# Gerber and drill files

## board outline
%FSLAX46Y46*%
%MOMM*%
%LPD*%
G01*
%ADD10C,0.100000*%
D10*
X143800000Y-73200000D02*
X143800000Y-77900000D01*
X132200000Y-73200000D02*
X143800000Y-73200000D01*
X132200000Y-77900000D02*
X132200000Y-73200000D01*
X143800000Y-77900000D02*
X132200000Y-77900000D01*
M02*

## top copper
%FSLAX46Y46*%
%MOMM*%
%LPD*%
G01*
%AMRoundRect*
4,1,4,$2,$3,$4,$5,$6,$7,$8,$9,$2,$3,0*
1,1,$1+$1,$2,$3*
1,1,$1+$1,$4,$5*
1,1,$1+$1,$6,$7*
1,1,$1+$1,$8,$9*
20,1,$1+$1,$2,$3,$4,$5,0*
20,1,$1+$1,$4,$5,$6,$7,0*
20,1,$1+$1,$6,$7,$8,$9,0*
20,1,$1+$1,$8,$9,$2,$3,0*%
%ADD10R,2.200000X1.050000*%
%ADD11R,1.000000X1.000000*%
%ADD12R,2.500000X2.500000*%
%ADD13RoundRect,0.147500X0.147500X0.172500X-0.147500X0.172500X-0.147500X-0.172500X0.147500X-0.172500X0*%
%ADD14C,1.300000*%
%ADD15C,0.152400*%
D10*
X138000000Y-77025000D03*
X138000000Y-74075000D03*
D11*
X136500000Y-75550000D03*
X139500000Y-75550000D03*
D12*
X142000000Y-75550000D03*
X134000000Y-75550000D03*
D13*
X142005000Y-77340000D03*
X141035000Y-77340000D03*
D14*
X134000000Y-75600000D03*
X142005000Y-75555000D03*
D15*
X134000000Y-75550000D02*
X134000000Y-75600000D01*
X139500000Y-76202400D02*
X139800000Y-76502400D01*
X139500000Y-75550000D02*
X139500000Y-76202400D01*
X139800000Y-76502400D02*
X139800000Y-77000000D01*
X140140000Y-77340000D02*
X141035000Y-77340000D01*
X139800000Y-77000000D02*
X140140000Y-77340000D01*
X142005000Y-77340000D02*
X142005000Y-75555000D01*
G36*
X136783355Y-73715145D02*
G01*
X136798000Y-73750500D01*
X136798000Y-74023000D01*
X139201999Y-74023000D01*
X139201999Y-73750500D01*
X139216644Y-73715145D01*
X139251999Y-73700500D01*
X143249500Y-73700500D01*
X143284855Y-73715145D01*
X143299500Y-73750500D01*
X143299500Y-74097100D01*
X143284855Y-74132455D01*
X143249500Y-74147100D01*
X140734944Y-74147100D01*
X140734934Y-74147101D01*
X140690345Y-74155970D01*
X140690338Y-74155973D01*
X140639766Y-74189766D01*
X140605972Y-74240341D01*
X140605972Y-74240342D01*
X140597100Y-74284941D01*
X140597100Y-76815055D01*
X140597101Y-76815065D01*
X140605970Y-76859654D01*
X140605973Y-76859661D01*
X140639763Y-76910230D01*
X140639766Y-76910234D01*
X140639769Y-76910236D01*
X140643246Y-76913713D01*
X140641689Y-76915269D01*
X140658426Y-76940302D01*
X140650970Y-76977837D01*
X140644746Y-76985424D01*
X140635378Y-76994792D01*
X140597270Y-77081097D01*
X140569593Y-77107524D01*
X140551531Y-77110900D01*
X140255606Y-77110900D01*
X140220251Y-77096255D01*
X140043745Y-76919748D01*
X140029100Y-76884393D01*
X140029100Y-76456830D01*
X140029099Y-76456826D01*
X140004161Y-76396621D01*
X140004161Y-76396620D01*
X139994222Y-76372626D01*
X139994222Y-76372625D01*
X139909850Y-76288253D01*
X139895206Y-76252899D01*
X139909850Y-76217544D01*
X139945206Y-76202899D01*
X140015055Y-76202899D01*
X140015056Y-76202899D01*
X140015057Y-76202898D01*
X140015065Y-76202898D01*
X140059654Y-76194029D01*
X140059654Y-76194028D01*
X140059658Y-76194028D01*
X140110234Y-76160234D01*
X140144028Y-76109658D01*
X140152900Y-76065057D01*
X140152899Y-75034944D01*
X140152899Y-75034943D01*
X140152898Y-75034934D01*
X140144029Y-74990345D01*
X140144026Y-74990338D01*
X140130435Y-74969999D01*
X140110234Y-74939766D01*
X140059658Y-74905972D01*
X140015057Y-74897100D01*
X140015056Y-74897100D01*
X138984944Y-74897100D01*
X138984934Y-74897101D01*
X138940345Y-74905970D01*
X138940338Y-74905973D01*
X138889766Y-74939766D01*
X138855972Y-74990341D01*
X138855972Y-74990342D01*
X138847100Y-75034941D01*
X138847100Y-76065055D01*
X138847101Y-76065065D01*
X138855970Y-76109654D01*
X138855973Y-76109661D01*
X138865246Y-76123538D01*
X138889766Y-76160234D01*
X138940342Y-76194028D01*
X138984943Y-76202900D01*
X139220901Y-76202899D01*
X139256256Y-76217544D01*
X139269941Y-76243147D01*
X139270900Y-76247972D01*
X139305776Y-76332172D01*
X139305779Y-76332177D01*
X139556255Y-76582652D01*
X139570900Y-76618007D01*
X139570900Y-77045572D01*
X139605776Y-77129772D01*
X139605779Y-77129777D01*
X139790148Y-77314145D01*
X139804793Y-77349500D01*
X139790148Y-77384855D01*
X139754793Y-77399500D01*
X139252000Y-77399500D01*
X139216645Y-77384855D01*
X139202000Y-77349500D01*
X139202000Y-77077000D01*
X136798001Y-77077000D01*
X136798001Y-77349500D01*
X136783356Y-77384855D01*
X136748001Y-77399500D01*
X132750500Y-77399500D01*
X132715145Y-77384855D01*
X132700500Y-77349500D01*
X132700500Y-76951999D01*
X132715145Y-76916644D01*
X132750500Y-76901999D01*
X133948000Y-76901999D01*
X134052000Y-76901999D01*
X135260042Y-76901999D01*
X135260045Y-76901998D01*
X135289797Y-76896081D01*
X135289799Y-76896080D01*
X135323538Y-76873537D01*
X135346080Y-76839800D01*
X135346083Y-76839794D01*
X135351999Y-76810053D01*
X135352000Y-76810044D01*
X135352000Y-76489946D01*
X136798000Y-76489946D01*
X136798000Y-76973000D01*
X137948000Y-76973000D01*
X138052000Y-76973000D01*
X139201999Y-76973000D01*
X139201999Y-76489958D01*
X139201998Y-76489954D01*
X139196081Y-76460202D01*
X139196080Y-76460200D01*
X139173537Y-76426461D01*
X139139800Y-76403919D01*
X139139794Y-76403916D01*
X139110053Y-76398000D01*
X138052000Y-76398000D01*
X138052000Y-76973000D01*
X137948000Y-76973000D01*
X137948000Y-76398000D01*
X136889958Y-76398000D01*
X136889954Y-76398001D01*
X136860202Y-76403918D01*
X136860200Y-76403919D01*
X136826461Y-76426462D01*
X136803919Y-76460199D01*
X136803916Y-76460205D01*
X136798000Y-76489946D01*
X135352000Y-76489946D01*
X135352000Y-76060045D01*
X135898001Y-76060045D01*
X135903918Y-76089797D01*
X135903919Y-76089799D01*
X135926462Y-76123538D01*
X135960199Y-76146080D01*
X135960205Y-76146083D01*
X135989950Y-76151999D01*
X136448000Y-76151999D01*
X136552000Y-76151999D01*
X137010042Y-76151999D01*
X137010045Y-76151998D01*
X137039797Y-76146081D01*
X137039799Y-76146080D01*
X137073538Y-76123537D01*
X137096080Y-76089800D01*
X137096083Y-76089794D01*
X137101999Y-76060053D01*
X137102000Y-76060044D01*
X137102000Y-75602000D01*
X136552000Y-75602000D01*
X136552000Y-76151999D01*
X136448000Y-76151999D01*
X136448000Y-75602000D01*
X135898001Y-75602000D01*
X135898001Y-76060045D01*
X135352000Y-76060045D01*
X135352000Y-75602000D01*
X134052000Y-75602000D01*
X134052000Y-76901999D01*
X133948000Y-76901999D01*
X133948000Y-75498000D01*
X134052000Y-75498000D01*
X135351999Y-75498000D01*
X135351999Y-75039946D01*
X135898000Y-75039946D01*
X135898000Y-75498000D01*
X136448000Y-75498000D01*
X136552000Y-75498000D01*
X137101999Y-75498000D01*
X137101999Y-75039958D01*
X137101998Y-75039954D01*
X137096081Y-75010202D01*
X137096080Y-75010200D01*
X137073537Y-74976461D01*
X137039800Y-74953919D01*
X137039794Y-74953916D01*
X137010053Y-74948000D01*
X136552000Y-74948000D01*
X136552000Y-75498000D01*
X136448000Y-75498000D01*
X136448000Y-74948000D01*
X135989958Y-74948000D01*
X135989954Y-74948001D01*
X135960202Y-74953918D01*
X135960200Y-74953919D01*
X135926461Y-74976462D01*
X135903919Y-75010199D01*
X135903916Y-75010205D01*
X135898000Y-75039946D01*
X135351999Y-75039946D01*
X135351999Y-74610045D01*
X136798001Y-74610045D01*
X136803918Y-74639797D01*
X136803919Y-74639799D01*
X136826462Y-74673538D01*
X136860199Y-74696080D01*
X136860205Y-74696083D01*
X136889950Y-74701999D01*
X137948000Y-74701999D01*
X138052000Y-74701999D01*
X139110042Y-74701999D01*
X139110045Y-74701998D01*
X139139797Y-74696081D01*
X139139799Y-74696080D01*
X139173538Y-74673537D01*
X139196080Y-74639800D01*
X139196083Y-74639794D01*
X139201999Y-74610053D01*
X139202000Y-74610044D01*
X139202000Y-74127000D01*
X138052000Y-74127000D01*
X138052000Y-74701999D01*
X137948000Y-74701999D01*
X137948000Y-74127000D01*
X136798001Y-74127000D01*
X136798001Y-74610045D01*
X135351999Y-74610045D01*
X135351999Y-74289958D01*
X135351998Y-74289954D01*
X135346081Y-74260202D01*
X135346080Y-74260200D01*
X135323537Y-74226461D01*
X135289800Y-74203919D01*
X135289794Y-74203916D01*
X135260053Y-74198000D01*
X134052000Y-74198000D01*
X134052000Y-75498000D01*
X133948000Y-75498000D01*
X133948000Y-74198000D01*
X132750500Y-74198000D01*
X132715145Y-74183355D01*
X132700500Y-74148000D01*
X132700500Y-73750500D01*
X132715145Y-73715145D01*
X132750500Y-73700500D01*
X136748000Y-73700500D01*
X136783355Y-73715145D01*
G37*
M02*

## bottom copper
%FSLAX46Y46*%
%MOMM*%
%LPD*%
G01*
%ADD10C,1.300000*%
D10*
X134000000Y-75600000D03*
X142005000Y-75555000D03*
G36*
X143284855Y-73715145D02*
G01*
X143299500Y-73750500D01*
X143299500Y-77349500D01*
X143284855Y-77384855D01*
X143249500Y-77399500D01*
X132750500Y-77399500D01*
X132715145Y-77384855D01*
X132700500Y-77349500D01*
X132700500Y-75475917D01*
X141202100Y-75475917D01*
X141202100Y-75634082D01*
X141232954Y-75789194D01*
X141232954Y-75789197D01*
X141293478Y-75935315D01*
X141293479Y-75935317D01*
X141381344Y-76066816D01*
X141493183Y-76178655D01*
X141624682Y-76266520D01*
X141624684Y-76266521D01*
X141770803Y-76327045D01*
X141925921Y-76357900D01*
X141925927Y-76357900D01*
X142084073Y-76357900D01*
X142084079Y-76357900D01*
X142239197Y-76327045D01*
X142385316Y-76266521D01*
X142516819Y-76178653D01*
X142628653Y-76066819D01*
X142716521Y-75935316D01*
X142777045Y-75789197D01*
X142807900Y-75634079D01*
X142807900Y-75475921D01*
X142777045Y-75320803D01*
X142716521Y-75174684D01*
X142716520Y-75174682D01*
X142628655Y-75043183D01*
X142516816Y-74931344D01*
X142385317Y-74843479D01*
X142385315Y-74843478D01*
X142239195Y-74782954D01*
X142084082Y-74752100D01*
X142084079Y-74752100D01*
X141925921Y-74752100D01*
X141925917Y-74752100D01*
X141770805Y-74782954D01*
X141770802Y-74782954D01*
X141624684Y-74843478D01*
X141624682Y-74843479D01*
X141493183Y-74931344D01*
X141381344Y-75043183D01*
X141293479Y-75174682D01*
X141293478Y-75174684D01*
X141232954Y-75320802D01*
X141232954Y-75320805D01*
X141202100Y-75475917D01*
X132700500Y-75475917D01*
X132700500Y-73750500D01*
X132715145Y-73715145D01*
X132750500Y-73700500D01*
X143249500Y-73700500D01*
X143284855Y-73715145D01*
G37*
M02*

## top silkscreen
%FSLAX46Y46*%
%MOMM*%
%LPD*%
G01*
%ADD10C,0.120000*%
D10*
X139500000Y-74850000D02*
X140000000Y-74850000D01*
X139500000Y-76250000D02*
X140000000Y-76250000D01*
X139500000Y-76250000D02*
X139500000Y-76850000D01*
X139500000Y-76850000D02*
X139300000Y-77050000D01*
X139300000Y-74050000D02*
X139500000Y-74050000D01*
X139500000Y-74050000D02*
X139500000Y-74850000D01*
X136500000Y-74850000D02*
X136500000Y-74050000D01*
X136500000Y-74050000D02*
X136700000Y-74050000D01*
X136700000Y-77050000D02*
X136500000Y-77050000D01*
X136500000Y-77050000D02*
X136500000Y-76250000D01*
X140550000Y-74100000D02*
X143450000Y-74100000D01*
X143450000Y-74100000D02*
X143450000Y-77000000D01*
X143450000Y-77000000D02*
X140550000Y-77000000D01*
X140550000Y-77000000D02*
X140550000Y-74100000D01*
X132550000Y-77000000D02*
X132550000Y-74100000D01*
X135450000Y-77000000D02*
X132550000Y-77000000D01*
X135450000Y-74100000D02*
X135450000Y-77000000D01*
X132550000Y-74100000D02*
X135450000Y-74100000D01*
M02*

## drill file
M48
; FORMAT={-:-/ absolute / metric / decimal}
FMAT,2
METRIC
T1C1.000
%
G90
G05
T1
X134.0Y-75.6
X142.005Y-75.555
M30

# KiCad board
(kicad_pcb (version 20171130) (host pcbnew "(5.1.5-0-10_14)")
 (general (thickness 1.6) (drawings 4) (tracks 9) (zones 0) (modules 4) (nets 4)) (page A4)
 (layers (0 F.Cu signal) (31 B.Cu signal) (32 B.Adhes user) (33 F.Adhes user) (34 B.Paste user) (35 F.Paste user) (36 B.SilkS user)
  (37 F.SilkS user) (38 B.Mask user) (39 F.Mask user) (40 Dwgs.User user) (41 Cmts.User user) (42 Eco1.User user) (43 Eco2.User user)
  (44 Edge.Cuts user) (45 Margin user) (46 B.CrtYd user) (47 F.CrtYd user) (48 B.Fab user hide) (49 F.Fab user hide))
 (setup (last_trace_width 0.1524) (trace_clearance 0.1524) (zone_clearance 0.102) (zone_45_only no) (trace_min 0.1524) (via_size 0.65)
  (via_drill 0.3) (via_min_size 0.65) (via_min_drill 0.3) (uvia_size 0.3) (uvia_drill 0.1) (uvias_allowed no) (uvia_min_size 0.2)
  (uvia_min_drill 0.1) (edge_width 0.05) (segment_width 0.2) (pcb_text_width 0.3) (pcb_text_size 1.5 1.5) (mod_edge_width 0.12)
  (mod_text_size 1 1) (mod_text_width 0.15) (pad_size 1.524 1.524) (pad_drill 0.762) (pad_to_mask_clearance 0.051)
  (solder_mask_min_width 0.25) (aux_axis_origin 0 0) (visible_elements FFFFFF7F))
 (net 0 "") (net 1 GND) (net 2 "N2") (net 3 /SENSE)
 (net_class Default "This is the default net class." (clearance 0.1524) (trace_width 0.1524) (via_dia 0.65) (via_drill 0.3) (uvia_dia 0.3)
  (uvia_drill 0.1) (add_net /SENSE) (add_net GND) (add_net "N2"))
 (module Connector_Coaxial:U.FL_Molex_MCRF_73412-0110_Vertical (layer F.Cu) (at 138 75.55 90)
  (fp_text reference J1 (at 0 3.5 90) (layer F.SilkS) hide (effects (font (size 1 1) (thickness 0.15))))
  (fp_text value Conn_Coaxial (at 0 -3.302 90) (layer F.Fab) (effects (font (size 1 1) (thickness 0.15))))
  (fp_line (start 0.7 1.5) (end 0.7 2) (layer F.SilkS) (width 0.12))
  (fp_line (start -0.7 1.5) (end -0.7 2) (layer F.SilkS) (width 0.12))
  (fp_line (start -0.7 1.5) (end -1.3 1.5) (layer F.SilkS) (width 0.12))
  (fp_line (start -1.3 1.5) (end -1.5 1.3) (layer F.SilkS) (width 0.12))
  (fp_line (start 1.5 1.3) (end 1.5 1.5) (layer F.SilkS) (width 0.12))
  (fp_line (start 1.5 1.5) (end 0.7 1.5) (layer F.SilkS) (width 0.12))
  (fp_line (start 0.7 -1.5) (end 1.5 -1.5) (layer F.SilkS) (width 0.12))
  (fp_line (start 1.5 -1.5) (end 1.5 -1.3) (layer F.SilkS) (width 0.12))
  (fp_line (start -1.5 -1.3) (end -1.5 -1.5) (layer F.SilkS) (width 0.12))
  (fp_line (start -1.5 -1.5) (end -0.7 -1.5) (layer F.SilkS) (width 0.12))
  (pad 2 smd rect (at -1.475 0 90) (size 1.05 2.2) (layers F.Cu F.Paste F.Mask) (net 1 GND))
  (pad 2 smd rect (at 1.475 0 90) (size 1.05 2.2) (layers F.Cu F.Paste F.Mask) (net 1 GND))
  (pad 2 smd rect (at 0 -1.5 90) (size 1 1) (layers F.Cu F.Paste F.Mask) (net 1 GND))
  (pad 1 smd rect (at 0 1.5 90) (size 1 1) (layers F.Cu F.Paste F.Mask) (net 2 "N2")))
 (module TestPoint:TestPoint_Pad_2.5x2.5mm (layer F.Cu) (at 142 75.55)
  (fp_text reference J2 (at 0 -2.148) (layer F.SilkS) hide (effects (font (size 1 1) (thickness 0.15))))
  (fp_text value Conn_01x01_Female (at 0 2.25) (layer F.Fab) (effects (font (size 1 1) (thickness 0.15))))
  (fp_line (start -1.45 -1.45) (end 1.45 -1.45) (layer F.SilkS) (width 0.12))
  (fp_line (start 1.45 -1.45) (end 1.45 1.45) (layer F.SilkS) (width 0.12))
  (fp_line (start 1.45 1.45) (end -1.45 1.45) (layer F.SilkS) (width 0.12))
  (fp_line (start -1.45 1.45) (end -1.45 -1.45) (layer F.SilkS) (width 0.12))
  (pad 1 smd rect (at 0 0) (size 2.5 2.5) (layers F.Cu F.Mask) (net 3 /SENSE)))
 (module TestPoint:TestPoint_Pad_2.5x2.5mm (layer F.Cu) (at 134 75.55)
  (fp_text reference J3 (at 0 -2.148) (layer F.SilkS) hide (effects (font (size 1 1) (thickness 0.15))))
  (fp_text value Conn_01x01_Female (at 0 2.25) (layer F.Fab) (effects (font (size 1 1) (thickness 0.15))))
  (fp_line (start -1.45 1.45) (end -1.45 -1.45) (layer F.SilkS) (width 0.12))
  (fp_line (start 1.45 1.45) (end -1.45 1.45) (layer F.SilkS) (width 0.12))
  (fp_line (start 1.45 -1.45) (end 1.45 1.45) (layer F.SilkS) (width 0.12))
  (fp_line (start -1.45 -1.45) (end 1.45 -1.45) (layer F.SilkS) (width 0.12))
  (pad 1 smd rect (at 0 0) (size 2.5 2.5) (layers F.Cu F.Mask) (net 1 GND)))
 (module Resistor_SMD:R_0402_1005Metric (layer F.Cu) (at 141.52 77.34 180)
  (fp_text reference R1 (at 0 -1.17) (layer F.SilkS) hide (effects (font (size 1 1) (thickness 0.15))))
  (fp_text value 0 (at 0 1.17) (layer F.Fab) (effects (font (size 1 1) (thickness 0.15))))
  (pad 1 smd roundrect (at -0.485 0 180) (size 0.59 0.64) (layers F.Cu F.Paste F.Mask) (roundrect_rratio 0.25) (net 3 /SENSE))
  (pad 2 smd roundrect (at 0.485 0 180) (size 0.59 0.64) (layers F.Cu F.Paste F.Mask) (roundrect_rratio 0.25) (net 2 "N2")))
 (gr_line (start 143.8 73.2) (end 143.8 77.9) (layer Edge.Cuts) (width 0.1))
 (gr_line (start 132.2 73.2) (end 143.8 73.2) (layer Edge.Cuts) (width 0.1))
 (gr_line (start 132.2 77.9) (end 132.2 73.2) (layer Edge.Cuts) (width 0.1))
 (gr_line (start 143.8 77.9) (end 132.2 77.9) (layer Edge.Cuts) (width 0.1))
 (via (at 134 75.6) (size 1.3) (drill 1) (layers F.Cu B.Cu) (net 1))
 (segment (start 134 75.55) (end 134 75.6) (width 0.1524) (layer F.Cu) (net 1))
 (segment (start 139.5 76.2024) (end 139.8 76.5024) (width 0.1524) (layer F.Cu) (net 2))
 (segment (start 139.5 75.55) (end 139.5 76.2024) (width 0.1524) (layer F.Cu) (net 2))
 (segment (start 139.8 76.5024) (end 139.8 77) (width 0.1524) (layer F.Cu) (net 2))
 (segment (start 140.14 77.34) (end 141.035 77.34) (width 0.1524) (layer F.Cu) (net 2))
 (segment (start 139.8 77) (end 140.14 77.34) (width 0.1524) (layer F.Cu) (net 2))
 (segment (start 142.005 77.34) (end 142.005 75.555) (width 0.1524) (layer F.Cu) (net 3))
 (via (at 142.005 75.555) (size 1.3) (drill 1) (layers F.Cu B.Cu) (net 3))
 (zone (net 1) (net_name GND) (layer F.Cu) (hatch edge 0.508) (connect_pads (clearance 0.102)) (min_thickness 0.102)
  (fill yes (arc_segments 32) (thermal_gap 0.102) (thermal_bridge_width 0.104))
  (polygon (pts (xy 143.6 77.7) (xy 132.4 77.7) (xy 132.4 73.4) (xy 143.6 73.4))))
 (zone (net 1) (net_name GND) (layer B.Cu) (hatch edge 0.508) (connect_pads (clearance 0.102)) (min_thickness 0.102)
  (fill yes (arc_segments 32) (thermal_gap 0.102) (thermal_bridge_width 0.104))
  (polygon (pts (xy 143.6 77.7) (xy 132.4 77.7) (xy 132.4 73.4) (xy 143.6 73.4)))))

